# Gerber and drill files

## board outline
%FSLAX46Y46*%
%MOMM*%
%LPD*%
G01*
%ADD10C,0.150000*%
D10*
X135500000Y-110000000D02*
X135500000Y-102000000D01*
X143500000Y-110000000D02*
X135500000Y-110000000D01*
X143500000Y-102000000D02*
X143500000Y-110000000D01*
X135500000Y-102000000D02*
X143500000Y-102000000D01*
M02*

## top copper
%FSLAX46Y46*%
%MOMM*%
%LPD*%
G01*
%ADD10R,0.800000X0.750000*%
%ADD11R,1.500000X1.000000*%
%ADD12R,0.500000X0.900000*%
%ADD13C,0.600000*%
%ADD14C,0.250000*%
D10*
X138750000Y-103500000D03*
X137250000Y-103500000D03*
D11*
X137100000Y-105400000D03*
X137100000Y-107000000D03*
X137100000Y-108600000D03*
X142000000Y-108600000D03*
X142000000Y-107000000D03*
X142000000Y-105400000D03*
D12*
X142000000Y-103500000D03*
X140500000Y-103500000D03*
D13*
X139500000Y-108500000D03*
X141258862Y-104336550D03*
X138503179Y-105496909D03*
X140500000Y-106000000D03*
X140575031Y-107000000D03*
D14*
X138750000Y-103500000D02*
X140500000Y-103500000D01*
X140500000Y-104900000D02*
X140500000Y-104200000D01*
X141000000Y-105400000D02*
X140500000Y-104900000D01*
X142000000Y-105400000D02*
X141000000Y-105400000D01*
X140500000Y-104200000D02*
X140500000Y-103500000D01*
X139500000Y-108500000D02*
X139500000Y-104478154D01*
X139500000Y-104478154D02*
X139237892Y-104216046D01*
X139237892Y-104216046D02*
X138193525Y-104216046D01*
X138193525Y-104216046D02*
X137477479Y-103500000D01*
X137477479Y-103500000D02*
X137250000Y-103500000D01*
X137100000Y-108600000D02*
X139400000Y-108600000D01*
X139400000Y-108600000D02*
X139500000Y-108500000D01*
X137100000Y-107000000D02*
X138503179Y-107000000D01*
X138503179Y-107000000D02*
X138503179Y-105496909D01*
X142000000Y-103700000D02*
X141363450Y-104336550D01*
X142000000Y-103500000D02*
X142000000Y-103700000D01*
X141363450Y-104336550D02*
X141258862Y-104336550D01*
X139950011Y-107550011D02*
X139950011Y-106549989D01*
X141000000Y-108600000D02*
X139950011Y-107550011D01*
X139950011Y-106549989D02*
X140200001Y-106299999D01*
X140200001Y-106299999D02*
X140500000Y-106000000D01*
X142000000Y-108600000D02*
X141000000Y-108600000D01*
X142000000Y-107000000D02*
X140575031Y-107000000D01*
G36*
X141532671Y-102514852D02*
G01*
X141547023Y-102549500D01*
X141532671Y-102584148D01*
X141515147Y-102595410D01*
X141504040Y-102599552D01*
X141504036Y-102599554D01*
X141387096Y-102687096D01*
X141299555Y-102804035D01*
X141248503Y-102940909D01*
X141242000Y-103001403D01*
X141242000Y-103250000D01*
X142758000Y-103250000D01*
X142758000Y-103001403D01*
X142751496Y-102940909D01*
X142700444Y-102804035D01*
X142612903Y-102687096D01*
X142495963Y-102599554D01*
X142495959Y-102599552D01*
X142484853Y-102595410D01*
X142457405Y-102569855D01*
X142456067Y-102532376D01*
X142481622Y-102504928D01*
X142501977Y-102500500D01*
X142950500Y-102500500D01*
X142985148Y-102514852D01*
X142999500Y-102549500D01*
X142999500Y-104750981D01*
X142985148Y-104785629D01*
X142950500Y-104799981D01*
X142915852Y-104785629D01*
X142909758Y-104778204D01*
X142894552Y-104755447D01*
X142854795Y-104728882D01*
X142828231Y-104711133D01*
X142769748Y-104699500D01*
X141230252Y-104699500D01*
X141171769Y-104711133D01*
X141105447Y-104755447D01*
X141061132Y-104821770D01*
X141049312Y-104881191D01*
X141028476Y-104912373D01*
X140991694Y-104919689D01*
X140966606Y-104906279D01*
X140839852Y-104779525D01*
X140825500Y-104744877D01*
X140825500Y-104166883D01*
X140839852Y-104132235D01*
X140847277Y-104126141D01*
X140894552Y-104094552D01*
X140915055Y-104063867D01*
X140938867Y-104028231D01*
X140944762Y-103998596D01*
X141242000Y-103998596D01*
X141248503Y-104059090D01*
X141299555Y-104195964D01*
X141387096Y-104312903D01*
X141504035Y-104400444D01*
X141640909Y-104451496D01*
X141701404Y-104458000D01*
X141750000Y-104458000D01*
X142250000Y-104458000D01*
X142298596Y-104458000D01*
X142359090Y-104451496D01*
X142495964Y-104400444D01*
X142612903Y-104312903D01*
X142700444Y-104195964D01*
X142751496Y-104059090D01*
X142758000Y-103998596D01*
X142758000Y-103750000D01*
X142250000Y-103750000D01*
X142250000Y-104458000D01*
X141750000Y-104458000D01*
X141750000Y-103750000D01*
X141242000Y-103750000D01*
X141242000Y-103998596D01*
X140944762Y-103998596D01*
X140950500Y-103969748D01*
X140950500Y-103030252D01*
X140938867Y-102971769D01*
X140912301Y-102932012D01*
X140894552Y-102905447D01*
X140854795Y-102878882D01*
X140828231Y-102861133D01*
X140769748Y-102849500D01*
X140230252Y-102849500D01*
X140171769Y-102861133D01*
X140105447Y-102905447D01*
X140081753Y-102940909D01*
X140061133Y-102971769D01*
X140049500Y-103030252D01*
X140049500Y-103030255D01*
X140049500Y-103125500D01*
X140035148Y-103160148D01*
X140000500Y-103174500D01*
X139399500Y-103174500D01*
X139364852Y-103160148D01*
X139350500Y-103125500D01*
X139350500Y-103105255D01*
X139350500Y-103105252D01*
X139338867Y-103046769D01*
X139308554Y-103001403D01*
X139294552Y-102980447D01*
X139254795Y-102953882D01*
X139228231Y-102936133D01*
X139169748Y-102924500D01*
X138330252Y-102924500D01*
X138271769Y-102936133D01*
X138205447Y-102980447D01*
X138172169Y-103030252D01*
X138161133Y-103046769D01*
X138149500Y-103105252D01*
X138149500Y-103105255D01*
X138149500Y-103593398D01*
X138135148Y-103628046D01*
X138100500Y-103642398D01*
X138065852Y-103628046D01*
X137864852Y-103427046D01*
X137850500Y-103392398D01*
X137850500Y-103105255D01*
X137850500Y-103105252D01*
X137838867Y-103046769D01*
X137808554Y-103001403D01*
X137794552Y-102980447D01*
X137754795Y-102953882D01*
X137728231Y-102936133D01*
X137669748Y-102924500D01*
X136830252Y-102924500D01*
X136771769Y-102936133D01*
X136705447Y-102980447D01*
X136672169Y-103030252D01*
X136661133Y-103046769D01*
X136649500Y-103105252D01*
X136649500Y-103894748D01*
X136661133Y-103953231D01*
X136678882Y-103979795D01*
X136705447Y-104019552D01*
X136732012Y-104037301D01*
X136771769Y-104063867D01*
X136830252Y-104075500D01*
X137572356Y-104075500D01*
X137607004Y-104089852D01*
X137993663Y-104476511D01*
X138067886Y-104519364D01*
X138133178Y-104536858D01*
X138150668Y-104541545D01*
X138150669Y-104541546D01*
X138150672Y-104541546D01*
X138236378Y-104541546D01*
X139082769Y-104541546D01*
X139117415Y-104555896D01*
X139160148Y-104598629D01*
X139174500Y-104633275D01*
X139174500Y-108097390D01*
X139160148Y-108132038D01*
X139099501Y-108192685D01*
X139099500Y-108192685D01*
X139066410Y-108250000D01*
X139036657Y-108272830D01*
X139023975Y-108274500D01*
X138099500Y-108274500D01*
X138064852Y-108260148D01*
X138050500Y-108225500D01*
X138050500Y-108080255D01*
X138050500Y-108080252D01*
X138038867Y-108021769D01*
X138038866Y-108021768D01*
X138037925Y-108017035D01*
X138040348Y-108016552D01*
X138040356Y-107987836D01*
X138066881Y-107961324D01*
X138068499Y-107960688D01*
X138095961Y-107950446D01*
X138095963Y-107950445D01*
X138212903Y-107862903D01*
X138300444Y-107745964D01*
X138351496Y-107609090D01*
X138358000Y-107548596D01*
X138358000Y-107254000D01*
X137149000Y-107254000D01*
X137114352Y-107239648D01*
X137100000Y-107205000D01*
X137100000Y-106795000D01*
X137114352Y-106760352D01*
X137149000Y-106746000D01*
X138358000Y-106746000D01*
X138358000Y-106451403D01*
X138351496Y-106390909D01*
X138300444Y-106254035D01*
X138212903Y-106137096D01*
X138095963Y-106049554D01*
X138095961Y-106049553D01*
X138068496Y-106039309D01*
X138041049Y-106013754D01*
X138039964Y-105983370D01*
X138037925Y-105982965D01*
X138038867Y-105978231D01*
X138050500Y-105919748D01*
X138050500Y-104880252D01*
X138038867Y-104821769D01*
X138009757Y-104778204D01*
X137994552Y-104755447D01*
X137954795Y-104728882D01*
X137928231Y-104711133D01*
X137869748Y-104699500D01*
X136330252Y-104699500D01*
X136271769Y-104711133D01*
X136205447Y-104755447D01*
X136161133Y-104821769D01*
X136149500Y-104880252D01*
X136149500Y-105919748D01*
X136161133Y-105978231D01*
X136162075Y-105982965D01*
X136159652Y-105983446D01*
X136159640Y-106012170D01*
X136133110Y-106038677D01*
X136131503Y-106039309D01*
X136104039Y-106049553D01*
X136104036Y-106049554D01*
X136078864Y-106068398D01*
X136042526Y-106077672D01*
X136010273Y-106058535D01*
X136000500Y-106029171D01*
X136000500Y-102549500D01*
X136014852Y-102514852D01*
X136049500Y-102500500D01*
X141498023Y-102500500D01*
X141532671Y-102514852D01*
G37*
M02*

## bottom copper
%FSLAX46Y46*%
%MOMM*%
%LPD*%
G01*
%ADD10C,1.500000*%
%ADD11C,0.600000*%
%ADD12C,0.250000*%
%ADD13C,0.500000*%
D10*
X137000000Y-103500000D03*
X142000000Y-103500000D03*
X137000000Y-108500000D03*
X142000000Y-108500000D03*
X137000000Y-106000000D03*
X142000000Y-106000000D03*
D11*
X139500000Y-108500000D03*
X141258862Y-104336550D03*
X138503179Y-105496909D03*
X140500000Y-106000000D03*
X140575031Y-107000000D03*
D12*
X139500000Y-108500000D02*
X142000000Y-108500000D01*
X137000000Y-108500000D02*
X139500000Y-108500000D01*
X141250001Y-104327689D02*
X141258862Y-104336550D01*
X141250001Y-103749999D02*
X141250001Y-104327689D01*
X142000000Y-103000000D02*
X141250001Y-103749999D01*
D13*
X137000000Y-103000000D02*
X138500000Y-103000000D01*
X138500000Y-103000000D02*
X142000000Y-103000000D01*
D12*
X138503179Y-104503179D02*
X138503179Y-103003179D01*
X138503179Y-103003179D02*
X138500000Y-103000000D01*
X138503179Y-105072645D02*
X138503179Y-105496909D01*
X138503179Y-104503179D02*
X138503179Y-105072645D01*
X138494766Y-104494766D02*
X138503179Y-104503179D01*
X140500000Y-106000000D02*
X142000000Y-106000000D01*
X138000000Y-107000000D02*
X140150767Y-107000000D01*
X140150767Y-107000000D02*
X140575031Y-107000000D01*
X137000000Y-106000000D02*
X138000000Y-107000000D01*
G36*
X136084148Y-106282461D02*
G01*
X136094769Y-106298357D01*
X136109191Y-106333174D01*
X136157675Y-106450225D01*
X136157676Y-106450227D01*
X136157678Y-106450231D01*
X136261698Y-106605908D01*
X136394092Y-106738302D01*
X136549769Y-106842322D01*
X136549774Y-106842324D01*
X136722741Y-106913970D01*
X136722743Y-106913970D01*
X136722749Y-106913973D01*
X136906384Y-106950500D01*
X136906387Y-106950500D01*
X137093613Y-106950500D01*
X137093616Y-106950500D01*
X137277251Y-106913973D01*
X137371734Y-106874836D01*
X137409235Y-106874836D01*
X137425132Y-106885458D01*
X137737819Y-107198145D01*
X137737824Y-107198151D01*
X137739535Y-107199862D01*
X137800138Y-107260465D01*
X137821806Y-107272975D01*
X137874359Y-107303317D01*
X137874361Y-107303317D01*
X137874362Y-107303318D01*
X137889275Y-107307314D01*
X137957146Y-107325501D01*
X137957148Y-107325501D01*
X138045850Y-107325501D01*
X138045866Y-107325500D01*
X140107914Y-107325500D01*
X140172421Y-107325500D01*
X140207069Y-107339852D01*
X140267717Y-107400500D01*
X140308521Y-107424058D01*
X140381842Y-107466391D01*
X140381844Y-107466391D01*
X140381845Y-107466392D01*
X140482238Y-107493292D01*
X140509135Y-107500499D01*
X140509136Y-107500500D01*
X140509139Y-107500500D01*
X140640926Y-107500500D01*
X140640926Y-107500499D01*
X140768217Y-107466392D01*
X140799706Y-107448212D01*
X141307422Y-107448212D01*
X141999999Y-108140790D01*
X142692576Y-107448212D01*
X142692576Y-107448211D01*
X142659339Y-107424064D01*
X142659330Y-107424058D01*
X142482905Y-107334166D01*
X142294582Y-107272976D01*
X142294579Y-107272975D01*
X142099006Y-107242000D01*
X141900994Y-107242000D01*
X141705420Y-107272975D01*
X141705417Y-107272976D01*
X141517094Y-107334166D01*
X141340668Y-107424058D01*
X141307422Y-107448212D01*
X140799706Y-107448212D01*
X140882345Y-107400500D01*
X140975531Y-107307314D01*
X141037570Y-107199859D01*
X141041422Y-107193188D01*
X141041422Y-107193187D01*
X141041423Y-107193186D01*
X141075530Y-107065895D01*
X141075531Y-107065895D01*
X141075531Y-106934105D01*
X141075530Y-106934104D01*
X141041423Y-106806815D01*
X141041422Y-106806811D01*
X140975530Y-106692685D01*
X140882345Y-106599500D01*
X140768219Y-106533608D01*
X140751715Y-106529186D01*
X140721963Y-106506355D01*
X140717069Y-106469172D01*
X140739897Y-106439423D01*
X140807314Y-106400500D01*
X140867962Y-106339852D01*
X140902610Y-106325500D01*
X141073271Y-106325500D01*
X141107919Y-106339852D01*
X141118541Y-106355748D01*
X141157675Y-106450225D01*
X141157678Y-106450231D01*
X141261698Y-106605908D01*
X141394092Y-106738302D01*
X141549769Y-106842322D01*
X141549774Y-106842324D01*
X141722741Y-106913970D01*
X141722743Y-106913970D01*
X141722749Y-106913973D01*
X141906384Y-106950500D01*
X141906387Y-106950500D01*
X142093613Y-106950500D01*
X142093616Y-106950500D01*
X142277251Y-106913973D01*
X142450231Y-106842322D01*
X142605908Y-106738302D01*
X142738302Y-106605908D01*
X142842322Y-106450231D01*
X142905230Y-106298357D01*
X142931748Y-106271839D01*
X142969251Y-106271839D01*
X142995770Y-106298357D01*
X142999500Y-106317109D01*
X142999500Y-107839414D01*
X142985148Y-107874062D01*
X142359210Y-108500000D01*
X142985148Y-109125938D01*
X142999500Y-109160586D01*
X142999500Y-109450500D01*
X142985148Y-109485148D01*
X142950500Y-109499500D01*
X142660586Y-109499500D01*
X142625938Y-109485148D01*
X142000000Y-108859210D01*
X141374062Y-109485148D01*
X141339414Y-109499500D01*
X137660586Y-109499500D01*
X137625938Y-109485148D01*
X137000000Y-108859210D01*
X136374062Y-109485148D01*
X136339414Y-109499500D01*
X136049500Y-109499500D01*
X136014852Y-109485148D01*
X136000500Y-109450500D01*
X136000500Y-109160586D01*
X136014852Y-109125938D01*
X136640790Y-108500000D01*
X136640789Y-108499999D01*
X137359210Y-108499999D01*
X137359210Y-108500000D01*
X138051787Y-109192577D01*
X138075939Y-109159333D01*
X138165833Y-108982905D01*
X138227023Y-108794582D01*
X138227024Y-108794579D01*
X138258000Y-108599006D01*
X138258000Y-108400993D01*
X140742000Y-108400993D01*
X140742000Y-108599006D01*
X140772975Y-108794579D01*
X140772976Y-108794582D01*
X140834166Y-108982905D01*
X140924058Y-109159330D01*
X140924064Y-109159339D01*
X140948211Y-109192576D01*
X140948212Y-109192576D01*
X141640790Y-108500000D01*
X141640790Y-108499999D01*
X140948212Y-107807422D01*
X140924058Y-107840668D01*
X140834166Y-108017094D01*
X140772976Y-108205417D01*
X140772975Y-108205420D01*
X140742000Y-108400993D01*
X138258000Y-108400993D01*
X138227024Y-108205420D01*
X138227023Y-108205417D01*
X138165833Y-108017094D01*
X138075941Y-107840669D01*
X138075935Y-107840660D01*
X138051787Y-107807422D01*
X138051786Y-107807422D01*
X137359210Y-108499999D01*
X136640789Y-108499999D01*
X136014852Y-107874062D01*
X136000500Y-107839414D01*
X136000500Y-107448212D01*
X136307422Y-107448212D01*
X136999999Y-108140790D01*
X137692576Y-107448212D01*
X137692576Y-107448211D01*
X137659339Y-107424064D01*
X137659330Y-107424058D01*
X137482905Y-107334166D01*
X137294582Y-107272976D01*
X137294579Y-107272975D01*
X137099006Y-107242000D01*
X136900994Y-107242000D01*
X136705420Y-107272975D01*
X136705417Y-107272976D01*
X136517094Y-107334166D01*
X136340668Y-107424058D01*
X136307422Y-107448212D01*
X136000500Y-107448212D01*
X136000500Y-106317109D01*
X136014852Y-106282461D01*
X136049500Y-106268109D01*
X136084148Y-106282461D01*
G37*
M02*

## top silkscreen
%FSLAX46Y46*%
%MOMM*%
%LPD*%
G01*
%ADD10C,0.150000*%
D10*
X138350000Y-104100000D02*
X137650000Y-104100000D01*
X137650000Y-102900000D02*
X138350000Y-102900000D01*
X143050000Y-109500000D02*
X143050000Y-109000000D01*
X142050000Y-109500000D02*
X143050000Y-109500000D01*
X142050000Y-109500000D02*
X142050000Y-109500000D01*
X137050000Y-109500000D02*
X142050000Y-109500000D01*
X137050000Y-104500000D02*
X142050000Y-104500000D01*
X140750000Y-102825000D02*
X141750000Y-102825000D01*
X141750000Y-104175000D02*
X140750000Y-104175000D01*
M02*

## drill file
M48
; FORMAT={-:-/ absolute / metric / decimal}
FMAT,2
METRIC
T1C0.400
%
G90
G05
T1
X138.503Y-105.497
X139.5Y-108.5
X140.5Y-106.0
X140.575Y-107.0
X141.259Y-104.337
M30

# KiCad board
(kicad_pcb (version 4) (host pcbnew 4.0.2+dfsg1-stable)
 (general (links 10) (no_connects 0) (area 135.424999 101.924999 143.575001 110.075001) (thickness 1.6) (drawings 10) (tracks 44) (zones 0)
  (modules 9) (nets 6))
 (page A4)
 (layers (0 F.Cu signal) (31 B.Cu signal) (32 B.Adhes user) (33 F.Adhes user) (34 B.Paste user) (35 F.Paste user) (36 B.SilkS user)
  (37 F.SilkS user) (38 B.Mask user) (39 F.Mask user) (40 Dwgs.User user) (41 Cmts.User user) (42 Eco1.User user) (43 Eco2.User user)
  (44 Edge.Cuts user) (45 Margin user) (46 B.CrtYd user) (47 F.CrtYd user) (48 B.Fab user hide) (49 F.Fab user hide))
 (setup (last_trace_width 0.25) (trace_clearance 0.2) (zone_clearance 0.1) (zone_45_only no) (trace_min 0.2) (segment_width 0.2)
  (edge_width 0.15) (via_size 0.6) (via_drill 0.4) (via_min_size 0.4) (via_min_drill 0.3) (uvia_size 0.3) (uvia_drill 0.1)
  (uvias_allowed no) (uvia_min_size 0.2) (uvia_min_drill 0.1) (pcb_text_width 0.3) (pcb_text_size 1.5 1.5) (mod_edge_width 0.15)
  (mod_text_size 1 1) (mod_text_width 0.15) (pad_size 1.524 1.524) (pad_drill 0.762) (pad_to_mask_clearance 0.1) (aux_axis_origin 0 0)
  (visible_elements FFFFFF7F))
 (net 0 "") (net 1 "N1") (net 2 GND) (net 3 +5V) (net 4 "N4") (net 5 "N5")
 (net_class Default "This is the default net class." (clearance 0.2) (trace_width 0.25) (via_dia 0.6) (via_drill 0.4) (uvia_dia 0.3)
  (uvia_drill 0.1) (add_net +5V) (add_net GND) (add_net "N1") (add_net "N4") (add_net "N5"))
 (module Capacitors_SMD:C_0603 (layer F.Cu) (at 138 103.5 180)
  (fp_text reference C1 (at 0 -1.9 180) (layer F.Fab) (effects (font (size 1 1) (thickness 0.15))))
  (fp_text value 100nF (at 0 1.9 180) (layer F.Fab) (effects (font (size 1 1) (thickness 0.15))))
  (fp_line (start -0.35 -0.6) (end 0.35 -0.6) (layer F.SilkS) (width 0.15))
  (fp_line (start 0.35 0.6) (end -0.35 0.6) (layer F.SilkS) (width 0.15))
  (pad 1 smd rect (at -0.75 0 180) (size 0.8 0.75) (layers F.Cu F.Paste F.Mask) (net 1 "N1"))
  (pad 2 smd rect (at 0.75 0 180) (size 0.8 0.75) (layers F.Cu F.Paste F.Mask) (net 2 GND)))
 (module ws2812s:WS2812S (layer F.Cu) (at 139.55 107)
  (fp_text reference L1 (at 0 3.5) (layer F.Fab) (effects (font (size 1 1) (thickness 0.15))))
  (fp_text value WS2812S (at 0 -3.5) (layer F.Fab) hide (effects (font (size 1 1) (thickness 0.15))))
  (fp_line (start 3.5 2.5) (end 3.5 2) (layer F.SilkS) (width 0.15))
  (fp_line (start 2.5 2.5) (end 3.5 2.5) (layer F.SilkS) (width 0.15))
  (fp_line (start 2.5 2.5) (end 2.5 2.5) (layer F.SilkS) (width 0.15))
  (fp_line (start -2.5 2.5) (end 2.5 2.5) (layer F.SilkS) (width 0.15))
  (fp_line (start -2.5 -2.5) (end 2.5 -2.5) (layer F.SilkS) (width 0.15))
  (pad 4 smd rect (at -2.45 -1.6) (size 1.5 1) (layers F.Cu F.Paste F.Mask))
  (pad 5 smd rect (at -2.45 0) (size 1.5 1) (layers F.Cu F.Paste F.Mask) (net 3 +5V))
  (pad 6 smd rect (at -2.45 1.6) (size 1.5 1) (layers F.Cu F.Paste F.Mask) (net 2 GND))
  (pad 1 smd rect (at 2.45 1.6) (size 1.5 1) (layers F.Cu F.Paste F.Mask) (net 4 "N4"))
  (pad 2 smd rect (at 2.45 0) (size 1.5 1) (layers F.Cu F.Paste F.Mask) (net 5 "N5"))
  (pad 3 smd rect (at 2.45 -1.6) (size 1.5 1) (layers F.Cu F.Paste F.Mask) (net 1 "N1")))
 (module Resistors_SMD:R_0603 (layer F.Cu) (at 141.25 103.5 180)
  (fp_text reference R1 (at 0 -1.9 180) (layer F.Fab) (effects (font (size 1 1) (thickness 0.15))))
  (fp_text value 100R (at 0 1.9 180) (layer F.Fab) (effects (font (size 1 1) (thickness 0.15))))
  (fp_line (start 0.5 0.675) (end -0.5 0.675) (layer F.SilkS) (width 0.15))
  (fp_line (start -0.5 -0.675) (end 0.5 -0.675) (layer F.SilkS) (width 0.15))
  (pad 1 smd rect (at -0.75 0 180) (size 0.5 0.9) (layers F.Cu F.Paste F.Mask) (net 3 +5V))
  (pad 2 smd rect (at 0.75 0 180) (size 0.5 0.9) (layers F.Cu F.Paste F.Mask) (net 1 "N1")))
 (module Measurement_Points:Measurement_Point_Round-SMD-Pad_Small (layer B.Cu) (at 137 103.5)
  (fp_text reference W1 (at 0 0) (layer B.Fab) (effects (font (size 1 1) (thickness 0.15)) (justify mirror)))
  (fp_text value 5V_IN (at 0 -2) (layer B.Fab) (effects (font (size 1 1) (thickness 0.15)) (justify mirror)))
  (pad 1 smd circle (at 0 0) (size 1.5 1.5) (layers B.Cu B.Mask) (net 3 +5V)))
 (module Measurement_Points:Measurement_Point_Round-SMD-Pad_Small (layer B.Cu) (at 142 103.5)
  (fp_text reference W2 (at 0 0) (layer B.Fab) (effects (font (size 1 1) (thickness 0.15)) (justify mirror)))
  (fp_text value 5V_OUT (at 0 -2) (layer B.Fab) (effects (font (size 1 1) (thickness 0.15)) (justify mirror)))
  (pad 1 smd circle (at 0 0) (size 1.5 1.5) (layers B.Cu B.Mask) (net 3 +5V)))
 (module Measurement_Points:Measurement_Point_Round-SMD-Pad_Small (layer B.Cu) (at 137 108.5)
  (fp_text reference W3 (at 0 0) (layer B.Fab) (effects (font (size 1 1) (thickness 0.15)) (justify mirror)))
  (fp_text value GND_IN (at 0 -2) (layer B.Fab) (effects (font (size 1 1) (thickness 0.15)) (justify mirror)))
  (pad 1 smd circle (at 0 0) (size 1.5 1.5) (layers B.Cu B.Mask) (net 2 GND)))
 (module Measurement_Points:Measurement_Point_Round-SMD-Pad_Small (layer B.Cu) (at 142 108.5)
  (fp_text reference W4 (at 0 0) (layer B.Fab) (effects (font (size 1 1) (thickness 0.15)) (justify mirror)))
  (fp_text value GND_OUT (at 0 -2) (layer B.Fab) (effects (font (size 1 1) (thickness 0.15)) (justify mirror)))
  (pad 1 smd circle (at 0 0) (size 1.5 1.5) (layers B.Cu B.Mask) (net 2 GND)))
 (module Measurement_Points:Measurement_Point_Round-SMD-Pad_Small (layer B.Cu) (at 137 106)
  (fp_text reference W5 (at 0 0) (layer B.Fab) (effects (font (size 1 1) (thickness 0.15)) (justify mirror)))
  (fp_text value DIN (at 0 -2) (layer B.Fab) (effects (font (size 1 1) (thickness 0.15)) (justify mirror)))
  (pad 1 smd circle (at 0 0) (size 1.5 1.5) (layers B.Cu B.Mask) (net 5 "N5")))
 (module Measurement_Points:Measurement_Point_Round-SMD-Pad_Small (layer B.Cu) (at 142 106)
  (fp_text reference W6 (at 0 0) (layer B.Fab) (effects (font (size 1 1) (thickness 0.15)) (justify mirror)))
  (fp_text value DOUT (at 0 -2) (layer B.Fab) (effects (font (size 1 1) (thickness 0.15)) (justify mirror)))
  (pad 1 smd circle (at 0 0) (size 1.5 1.5) (layers B.Cu B.Mask) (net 4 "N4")))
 (gr_line (start 135.5 110) (end 135.5 102) (layer Edge.Cuts) (width 0.15))
 (gr_line (start 143.5 110) (end 135.5 110) (layer Edge.Cuts) (width 0.15))
 (gr_line (start 143.5 102) (end 143.5 110) (layer Edge.Cuts) (width 0.15))
 (gr_line (start 135.5 102) (end 143.5 102) (layer Edge.Cuts) (width 0.15))
 (segment (start 138.75 103.5) (end 140.5 103.5) (width 0.25) (layer F.Cu) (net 1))
 (segment (start 140.5 104.9) (end 140.5 104.2) (width 0.25) (layer F.Cu) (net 1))
 (segment (start 141 105.4) (end 140.5 104.9) (width 0.25) (layer F.Cu) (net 1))
 (segment (start 142 105.4) (end 141 105.4) (width 0.25) (layer F.Cu) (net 1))
 (segment (start 140.5 104.2) (end 140.5 103.5) (width 0.25) (layer F.Cu) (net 1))
 (segment (start 139.5 108.5) (end 139.5 104.478154) (width 0.25) (layer F.Cu) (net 2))
 (segment (start 139.5 104.478154) (end 139.237892 104.216046) (width 0.25) (layer F.Cu) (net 2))
 (segment (start 139.237892 104.216046) (end 138.193525 104.216046) (width 0.25) (layer F.Cu) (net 2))
 (segment (start 138.193525 104.216046) (end 137.477479 103.5) (width 0.25) (layer F.Cu) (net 2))
 (segment (start 137.477479 103.5) (end 137.25 103.5) (width 0.25) (layer F.Cu) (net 2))
 (segment (start 137.1 108.6) (end 139.4 108.6) (width 0.25) (layer F.Cu) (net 2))
 (segment (start 139.4 108.6) (end 139.5 108.5) (width 0.25) (layer F.Cu) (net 2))
 (segment (start 139.5 108.5) (end 142 108.5) (width 0.25) (layer B.Cu) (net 2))
 (segment (start 137 108.5) (end 139.5 108.5) (width 0.25) (layer B.Cu) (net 2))
 (via (at 139.5 108.5) (size 0.6) (drill 0.4) (layers F.Cu B.Cu) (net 2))
 (segment (start 137.1 107) (end 138.503179 107) (width 0.25) (layer F.Cu) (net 3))
 (segment (start 138.503179 107) (end 138.503179 105.496909) (width 0.25) (layer F.Cu) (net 3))
 (segment (start 142 103.7) (end 141.36345 104.33655) (width 0.25) (layer F.Cu) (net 3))
 (segment (start 142 103.5) (end 142 103.7) (width 0.25) (layer F.Cu) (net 3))
 (segment (start 141.250001 104.327689) (end 141.258862 104.33655) (width 0.25) (layer B.Cu) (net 3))
 (segment (start 141.36345 104.33655) (end 141.258862 104.33655) (width 0.25) (layer F.Cu) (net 3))
 (via (at 141.258862 104.33655) (size 0.6) (drill 0.4) (layers F.Cu B.Cu) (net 3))
 (segment (start 141.250001 103.749999) (end 141.250001 104.327689) (width 0.25) (layer B.Cu) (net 3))
 (segment (start 142 103) (end 141.250001 103.749999) (width 0.25) (layer B.Cu) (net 3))
 (segment (start 137 103) (end 138.5 103) (width 0.5) (layer B.Cu) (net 3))
 (segment (start 138.5 103) (end 142 103) (width 0.5) (layer B.Cu) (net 3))
 (segment (start 138.503179 104.503179) (end 138.503179 103.003179) (width 0.25) (layer B.Cu) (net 3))
 (segment (start 138.503179 103.003179) (end 138.5 103) (width 0.25) (layer B.Cu) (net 3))
 (segment (start 138.503179 105.072645) (end 138.503179 105.496909) (width 0.25) (layer B.Cu) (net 3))
 (segment (start 138.503179 104.503179) (end 138.503179 105.072645) (width 0.25) (layer B.Cu) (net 3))
 (segment (start 138.494766 104.494766) (end 138.503179 104.503179) (width 0.25) (layer B.Cu) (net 3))
 (via (at 138.503179 105.496909) (size 0.6) (drill 0.4) (layers F.Cu B.Cu) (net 3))
 (segment (start 139.950011 107.550011) (end 139.950011 106.549989) (width 0.25) (layer F.Cu) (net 4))
 (segment (start 141 108.6) (end 139.950011 107.550011) (width 0.25) (layer F.Cu) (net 4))
 (segment (start 139.950011 106.549989) (end 140.200001 106.299999) (width 0.25) (layer F.Cu) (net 4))
 (segment (start 140.200001 106.299999) (end 140.5 106) (width 0.25) (layer F.Cu) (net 4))
 (segment (start 142 108.6) (end 141 108.6) (width 0.25) (layer F.Cu) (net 4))
 (segment (start 140.5 106) (end 142 106) (width 0.25) (layer B.Cu) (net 4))
 (via (at 140.5 106) (size 0.6) (drill 0.4) (layers F.Cu B.Cu) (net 4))
 (segment (start 138 107) (end 140.150767 107) (width 0.25) (layer B.Cu) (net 5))
 (segment (start 140.150767 107) (end 140.575031 107) (width 0.25) (layer B.Cu) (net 5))
 (via (at 140.575031 107) (size 0.6) (drill 0.4) (layers F.Cu B.Cu) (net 5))
 (segment (start 142 107) (end 140.575031 107) (width 0.25) (layer F.Cu) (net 5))
 (segment (start 137 106) (end 138 107) (width 0.25) (layer B.Cu) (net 5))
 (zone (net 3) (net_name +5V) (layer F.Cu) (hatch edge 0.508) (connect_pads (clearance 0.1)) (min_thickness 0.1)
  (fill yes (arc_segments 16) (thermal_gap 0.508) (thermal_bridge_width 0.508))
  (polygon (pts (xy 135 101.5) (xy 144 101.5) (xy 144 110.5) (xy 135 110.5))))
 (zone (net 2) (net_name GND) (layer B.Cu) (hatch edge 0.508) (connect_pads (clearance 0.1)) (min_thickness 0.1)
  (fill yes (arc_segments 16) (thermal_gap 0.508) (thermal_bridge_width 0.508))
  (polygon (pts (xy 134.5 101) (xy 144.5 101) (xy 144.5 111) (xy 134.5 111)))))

